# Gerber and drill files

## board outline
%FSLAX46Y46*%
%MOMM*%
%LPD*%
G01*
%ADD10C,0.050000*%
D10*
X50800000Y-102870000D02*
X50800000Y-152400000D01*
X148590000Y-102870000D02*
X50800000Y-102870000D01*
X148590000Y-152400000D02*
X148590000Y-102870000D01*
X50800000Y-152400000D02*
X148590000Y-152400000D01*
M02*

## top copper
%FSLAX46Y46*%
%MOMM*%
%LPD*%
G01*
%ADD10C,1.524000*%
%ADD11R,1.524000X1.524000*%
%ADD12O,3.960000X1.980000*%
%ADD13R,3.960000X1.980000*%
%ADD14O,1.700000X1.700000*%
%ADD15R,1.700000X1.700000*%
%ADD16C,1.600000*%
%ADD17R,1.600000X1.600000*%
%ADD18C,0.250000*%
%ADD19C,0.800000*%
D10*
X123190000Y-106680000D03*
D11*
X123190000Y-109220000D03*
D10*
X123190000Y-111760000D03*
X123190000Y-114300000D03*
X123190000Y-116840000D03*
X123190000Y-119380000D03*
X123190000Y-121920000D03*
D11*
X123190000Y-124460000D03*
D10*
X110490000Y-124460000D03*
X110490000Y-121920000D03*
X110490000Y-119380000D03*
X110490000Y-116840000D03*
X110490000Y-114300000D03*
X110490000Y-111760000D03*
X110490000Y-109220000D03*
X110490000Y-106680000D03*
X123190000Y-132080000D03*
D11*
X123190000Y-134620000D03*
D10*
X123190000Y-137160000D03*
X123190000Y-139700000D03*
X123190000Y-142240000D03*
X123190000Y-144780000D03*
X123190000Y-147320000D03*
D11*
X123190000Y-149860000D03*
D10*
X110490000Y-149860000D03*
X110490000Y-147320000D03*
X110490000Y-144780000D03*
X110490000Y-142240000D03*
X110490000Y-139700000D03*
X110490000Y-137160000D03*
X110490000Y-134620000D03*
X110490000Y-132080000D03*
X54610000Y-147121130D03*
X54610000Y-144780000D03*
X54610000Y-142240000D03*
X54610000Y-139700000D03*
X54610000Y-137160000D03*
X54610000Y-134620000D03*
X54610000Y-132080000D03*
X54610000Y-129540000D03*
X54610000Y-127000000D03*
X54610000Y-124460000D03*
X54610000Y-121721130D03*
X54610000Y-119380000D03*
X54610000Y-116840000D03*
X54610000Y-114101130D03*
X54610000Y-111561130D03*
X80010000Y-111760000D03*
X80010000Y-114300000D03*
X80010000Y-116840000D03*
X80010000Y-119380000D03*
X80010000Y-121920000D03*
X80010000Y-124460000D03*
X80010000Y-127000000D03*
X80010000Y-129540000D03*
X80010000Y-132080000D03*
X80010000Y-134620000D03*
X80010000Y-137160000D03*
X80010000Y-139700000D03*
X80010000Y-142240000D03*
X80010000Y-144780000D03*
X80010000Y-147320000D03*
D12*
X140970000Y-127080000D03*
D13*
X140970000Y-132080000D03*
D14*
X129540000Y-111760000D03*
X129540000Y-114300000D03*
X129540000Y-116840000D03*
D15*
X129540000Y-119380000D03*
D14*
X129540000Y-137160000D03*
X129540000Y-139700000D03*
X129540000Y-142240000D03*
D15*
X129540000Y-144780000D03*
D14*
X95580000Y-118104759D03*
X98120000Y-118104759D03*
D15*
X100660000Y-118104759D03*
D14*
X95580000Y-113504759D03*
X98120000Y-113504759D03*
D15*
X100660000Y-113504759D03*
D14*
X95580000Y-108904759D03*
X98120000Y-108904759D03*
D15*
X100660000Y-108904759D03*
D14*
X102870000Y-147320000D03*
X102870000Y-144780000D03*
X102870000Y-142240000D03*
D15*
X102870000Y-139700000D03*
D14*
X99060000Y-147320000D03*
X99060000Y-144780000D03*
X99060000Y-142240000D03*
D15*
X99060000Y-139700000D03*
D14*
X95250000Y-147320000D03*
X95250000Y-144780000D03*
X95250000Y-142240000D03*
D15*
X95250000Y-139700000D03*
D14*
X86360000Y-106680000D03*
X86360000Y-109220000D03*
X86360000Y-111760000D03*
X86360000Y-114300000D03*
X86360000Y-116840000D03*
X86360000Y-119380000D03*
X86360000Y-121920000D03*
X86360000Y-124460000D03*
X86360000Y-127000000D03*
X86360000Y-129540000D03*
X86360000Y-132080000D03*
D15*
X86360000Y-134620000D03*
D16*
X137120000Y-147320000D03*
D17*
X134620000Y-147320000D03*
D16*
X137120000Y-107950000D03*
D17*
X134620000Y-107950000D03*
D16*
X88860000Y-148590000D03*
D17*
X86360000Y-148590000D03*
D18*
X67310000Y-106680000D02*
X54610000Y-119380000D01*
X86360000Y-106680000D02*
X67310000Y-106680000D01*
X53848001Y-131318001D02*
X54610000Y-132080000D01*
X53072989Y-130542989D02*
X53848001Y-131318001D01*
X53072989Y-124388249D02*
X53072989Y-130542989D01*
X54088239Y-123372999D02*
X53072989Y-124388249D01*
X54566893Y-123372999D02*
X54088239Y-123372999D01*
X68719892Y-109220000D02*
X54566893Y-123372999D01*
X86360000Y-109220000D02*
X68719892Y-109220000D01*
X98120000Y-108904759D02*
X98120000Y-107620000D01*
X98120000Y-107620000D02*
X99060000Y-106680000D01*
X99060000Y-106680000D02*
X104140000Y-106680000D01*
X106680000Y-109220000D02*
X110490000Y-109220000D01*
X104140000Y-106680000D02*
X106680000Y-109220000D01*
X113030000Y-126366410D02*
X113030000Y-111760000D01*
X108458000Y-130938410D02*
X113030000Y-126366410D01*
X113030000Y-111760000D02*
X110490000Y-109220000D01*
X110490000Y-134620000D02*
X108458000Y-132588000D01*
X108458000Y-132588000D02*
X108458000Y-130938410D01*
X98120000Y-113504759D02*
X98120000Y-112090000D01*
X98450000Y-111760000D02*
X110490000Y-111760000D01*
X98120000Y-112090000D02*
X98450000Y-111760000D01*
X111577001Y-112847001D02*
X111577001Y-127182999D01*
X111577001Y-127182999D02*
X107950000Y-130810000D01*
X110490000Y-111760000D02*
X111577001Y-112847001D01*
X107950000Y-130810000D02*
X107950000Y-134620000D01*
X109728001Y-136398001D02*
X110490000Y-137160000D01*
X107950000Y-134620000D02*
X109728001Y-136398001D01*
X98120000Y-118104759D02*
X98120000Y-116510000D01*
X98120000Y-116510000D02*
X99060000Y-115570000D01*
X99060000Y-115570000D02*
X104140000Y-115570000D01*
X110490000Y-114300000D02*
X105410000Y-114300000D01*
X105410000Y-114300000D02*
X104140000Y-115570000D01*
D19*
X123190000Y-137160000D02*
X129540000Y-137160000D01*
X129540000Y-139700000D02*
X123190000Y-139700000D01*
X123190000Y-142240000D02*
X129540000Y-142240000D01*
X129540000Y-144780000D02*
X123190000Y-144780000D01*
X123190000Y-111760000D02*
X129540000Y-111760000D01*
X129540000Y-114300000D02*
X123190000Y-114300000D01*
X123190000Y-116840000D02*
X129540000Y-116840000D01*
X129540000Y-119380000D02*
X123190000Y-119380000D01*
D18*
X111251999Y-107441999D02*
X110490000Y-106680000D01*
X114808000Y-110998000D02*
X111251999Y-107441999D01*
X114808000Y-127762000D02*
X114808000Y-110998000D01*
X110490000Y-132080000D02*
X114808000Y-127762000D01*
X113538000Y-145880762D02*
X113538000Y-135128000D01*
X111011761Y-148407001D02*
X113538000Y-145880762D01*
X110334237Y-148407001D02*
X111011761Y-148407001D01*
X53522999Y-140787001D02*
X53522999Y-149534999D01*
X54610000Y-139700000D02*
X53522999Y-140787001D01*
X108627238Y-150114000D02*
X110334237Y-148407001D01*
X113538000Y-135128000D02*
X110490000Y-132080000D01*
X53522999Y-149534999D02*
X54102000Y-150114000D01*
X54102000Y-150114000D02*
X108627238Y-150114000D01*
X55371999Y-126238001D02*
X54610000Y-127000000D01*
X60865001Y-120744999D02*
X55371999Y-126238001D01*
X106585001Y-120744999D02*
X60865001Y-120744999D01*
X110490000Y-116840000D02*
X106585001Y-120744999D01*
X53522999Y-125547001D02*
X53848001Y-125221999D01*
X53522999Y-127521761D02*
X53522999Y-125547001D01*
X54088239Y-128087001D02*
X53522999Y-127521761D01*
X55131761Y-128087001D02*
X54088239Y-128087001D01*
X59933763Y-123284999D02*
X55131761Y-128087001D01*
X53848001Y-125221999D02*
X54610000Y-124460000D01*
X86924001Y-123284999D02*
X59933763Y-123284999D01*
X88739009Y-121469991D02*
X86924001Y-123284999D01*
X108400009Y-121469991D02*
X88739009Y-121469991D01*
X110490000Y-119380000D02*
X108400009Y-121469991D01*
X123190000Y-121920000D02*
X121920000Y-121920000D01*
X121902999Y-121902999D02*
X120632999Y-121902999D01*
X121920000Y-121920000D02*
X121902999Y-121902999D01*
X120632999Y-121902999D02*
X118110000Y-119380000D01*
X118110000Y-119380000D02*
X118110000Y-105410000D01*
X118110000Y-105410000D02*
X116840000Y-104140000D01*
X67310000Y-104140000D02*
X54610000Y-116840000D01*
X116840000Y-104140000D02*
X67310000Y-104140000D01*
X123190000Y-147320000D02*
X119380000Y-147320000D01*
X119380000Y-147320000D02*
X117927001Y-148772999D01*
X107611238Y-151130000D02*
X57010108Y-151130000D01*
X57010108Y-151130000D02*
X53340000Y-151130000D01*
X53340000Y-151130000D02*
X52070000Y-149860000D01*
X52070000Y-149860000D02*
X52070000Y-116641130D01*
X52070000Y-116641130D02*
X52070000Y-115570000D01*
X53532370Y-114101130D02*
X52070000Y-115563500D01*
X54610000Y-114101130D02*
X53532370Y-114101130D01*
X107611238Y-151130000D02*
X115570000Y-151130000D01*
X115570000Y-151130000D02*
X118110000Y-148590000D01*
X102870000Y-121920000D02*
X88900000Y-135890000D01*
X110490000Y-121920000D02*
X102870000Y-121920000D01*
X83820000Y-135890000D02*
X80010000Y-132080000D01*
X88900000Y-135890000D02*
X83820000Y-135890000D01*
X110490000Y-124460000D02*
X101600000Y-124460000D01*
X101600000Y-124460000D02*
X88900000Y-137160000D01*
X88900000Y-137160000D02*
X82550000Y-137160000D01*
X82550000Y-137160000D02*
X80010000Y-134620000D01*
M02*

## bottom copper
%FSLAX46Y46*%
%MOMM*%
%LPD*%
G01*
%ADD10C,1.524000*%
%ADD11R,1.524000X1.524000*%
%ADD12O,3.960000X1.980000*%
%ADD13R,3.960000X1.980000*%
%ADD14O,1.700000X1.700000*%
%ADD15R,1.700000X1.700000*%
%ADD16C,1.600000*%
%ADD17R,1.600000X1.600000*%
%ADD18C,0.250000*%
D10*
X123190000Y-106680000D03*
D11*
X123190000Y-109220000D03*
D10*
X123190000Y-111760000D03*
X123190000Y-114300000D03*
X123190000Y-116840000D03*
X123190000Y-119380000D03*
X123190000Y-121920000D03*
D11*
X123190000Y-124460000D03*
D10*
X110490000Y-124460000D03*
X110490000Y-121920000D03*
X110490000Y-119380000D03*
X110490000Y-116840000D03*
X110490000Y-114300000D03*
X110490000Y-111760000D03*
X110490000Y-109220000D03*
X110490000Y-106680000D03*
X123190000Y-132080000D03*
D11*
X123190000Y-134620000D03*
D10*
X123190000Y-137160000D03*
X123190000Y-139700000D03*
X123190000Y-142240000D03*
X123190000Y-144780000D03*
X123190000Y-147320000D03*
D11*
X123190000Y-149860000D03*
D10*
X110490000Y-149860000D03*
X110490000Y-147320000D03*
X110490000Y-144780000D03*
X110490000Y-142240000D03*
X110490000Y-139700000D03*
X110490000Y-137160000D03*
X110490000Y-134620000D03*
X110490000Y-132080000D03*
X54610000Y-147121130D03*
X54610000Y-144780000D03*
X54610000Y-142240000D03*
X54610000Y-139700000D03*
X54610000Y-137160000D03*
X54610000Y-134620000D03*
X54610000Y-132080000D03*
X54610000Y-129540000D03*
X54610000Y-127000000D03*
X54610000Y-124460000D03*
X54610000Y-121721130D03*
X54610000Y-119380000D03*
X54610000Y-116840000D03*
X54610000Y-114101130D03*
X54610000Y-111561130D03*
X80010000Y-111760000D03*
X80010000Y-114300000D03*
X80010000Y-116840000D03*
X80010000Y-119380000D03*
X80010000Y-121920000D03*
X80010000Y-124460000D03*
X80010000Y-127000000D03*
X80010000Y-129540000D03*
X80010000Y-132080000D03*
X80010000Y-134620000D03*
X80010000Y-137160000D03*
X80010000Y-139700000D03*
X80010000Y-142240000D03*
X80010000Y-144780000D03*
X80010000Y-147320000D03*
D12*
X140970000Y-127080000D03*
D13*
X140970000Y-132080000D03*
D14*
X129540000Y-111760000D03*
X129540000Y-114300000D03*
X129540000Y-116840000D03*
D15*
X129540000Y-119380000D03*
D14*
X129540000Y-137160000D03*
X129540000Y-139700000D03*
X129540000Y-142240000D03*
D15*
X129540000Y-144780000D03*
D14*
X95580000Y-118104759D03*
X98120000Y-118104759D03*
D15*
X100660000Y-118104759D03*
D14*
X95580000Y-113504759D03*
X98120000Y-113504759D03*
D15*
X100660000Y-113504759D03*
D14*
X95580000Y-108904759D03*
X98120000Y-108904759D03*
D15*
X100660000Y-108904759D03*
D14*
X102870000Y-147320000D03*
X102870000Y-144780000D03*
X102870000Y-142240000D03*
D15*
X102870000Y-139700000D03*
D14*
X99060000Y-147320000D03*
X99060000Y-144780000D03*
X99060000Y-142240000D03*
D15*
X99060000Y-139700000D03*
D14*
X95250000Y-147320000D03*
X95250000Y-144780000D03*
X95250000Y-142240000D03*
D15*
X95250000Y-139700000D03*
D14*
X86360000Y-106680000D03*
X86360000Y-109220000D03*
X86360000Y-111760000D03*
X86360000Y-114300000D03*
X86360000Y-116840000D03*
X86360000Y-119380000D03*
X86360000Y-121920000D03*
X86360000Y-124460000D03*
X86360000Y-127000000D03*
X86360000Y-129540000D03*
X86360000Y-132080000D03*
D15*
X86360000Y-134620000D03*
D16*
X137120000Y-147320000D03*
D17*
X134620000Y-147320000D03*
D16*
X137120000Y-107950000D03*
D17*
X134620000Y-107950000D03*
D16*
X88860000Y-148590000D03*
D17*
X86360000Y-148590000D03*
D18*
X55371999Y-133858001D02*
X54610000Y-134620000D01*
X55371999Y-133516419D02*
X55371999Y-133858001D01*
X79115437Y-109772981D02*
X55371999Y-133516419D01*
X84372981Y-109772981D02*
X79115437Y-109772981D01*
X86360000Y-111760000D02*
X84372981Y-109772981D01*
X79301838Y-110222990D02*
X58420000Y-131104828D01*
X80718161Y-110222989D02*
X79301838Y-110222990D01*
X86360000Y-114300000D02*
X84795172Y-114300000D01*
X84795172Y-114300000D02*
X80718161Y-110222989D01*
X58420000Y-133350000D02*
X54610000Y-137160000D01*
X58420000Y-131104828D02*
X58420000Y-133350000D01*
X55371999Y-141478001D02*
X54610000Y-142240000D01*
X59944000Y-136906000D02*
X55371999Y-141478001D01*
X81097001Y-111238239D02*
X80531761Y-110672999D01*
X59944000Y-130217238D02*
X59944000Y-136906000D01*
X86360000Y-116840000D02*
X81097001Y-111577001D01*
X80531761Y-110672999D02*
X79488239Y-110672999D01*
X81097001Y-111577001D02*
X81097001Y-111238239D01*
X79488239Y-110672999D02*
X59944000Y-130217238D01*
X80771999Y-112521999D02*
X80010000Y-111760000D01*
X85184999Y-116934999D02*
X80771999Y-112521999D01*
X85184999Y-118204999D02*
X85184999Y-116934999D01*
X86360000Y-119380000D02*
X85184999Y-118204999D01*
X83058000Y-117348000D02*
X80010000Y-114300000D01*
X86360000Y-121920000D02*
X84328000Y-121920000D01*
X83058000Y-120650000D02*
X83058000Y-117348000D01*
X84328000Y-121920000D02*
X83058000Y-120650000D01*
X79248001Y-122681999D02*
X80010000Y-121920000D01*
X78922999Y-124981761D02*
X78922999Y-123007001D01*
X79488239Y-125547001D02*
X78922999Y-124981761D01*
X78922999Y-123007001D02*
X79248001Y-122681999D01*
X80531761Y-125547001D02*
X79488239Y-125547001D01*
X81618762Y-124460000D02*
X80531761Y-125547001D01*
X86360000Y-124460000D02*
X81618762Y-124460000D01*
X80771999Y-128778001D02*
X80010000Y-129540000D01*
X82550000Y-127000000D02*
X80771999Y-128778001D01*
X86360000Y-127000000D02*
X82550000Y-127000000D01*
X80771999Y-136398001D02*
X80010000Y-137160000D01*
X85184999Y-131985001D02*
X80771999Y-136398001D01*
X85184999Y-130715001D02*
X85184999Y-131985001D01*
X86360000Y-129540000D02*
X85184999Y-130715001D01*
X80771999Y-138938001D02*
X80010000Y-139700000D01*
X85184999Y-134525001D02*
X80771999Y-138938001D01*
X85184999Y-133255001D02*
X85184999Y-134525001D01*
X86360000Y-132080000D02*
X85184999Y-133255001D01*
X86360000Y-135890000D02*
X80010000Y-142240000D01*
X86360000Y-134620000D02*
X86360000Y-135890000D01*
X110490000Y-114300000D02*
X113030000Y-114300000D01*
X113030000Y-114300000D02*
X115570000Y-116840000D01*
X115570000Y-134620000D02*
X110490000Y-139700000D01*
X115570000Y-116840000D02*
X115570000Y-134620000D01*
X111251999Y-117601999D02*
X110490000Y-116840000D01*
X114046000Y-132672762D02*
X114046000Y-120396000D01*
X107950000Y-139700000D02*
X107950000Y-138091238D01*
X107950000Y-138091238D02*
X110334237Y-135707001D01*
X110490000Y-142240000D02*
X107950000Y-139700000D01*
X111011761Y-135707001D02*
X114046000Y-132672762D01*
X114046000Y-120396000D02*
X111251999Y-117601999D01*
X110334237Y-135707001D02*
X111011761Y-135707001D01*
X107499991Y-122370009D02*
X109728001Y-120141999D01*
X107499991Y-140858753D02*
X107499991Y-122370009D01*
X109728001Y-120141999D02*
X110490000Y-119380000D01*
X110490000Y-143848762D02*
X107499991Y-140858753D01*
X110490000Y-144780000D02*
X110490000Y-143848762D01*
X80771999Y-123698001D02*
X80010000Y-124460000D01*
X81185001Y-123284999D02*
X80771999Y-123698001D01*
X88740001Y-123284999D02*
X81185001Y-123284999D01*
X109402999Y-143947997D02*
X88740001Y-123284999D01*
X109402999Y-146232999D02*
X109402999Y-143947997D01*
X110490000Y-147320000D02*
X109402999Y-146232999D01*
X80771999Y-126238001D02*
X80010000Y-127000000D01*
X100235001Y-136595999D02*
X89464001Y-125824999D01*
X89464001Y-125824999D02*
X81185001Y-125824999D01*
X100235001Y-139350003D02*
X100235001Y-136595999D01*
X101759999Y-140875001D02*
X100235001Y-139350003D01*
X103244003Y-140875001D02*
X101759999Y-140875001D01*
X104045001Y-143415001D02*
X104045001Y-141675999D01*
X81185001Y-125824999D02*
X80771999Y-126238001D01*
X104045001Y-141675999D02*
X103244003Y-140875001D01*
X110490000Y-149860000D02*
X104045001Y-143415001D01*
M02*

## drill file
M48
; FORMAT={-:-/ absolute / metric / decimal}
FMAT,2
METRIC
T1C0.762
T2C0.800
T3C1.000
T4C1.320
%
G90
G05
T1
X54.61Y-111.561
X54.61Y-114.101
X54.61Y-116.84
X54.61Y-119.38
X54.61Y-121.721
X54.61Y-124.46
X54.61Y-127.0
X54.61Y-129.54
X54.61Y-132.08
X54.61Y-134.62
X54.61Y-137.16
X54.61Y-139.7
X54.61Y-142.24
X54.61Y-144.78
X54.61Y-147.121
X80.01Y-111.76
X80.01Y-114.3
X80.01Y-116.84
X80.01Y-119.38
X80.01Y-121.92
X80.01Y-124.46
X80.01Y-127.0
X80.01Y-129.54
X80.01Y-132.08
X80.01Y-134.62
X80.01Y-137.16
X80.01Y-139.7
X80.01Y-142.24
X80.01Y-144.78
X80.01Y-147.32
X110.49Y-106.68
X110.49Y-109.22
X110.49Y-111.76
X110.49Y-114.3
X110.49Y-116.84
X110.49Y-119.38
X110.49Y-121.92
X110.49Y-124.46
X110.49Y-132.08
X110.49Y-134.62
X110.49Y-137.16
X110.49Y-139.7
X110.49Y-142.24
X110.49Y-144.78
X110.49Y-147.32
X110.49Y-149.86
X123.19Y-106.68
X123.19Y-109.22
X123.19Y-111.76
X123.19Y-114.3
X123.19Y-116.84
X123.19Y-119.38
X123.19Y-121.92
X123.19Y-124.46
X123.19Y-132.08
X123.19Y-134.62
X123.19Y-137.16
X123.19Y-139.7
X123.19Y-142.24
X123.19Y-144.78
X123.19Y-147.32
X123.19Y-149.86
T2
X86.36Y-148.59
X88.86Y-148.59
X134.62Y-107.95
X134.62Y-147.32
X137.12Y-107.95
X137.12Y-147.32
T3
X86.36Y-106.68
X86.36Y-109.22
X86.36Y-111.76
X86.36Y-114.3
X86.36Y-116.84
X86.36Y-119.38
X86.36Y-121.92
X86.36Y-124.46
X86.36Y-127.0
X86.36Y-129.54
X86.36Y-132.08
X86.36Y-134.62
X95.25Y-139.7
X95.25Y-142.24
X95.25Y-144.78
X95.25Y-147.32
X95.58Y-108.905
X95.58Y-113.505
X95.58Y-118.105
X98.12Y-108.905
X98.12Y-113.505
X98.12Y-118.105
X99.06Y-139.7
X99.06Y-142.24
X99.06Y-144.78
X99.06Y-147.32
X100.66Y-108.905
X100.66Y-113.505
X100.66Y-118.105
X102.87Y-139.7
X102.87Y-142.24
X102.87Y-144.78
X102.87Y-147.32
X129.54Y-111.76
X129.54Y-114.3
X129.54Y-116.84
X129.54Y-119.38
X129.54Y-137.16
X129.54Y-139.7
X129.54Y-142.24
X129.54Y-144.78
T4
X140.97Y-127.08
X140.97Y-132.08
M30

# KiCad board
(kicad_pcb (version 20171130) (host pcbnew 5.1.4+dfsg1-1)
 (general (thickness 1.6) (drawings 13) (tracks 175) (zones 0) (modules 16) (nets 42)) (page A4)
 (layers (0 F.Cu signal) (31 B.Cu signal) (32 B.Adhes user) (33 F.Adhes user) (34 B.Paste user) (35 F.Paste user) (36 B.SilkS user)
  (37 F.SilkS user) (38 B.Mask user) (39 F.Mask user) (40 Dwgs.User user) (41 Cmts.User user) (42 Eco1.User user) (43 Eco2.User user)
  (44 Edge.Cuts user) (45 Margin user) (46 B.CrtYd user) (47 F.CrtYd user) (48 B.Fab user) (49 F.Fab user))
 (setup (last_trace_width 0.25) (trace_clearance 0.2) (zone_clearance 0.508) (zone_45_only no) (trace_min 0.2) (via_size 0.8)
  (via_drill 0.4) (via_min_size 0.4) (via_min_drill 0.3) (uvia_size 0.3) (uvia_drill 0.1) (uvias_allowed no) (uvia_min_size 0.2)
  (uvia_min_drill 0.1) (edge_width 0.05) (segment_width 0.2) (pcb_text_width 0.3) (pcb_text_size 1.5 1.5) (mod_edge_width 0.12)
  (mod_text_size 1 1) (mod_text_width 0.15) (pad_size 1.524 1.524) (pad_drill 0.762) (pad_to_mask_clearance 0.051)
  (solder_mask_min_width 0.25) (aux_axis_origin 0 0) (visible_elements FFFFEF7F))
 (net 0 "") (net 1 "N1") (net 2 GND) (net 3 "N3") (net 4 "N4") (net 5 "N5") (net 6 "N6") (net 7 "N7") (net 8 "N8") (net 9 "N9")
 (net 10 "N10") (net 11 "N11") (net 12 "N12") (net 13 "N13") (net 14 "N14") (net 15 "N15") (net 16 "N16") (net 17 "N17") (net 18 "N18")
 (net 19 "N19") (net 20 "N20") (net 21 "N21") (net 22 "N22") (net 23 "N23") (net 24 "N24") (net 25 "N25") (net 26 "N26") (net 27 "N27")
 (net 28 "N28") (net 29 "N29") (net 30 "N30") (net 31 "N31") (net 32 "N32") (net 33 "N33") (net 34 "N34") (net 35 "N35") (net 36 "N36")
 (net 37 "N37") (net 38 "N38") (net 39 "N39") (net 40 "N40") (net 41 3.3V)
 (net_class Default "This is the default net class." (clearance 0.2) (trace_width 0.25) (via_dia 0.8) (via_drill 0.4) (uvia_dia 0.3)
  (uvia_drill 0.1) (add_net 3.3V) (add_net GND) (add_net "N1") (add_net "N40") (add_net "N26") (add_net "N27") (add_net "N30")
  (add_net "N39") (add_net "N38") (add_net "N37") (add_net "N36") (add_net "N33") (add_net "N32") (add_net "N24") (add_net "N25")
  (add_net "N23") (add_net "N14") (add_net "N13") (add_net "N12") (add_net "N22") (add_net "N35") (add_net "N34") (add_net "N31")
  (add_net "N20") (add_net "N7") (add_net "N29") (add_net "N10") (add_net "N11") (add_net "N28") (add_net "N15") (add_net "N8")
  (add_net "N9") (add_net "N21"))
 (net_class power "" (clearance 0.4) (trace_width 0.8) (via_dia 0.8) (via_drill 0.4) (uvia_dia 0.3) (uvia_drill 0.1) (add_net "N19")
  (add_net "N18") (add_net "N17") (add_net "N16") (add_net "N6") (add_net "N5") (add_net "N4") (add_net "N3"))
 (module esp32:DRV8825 (layer F.Cu) (at 116.84 115.57)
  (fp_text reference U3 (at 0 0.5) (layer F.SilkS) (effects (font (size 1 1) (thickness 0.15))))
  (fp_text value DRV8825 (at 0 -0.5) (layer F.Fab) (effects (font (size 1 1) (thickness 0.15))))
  (pad 16 thru_hole circle (at 6.35 -8.89) (size 1.524 1.524) (drill 0.762) (layers *.Cu *.Mask) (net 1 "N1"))
  (pad 15 thru_hole rect (at 6.35 -6.35) (size 1.524 1.524) (drill 0.762) (layers *.Cu *.Mask) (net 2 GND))
  (pad 14 thru_hole circle (at 6.35 -3.81) (size 1.524 1.524) (drill 0.762) (layers *.Cu *.Mask) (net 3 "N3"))
  (pad 13 thru_hole circle (at 6.35 -1.27) (size 1.524 1.524) (drill 0.762) (layers *.Cu *.Mask) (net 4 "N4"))
  (pad 12 thru_hole circle (at 6.35 1.27) (size 1.524 1.524) (drill 0.762) (layers *.Cu *.Mask) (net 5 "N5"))
  (pad 11 thru_hole circle (at 6.35 3.81) (size 1.524 1.524) (drill 0.762) (layers *.Cu *.Mask) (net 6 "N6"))
  (pad 10 thru_hole circle (at 6.35 6.35) (size 1.524 1.524) (drill 0.762) (layers *.Cu *.Mask) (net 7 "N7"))
  (pad 9 thru_hole rect (at 6.35 8.89) (size 1.524 1.524) (drill 0.762) (layers *.Cu *.Mask) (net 2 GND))
  (pad 8 thru_hole circle (at -6.35 8.89) (size 1.524 1.524) (drill 0.762) (layers *.Cu *.Mask) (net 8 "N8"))
  (pad 7 thru_hole circle (at -6.35 6.35) (size 1.524 1.524) (drill 0.762) (layers *.Cu *.Mask) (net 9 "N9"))
  (pad 6 thru_hole circle (at -6.35 3.81) (size 1.524 1.524) (drill 0.762) (layers *.Cu *.Mask) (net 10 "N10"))
  (pad 5 thru_hole circle (at -6.35 1.27) (size 1.524 1.524) (drill 0.762) (layers *.Cu *.Mask) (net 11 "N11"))
  (pad 4 thru_hole circle (at -6.35 -1.27) (size 1.524 1.524) (drill 0.762) (layers *.Cu *.Mask) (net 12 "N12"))
  (pad 3 thru_hole circle (at -6.35 -3.81) (size 1.524 1.524) (drill 0.762) (layers *.Cu *.Mask) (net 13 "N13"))
  (pad 2 thru_hole circle (at -6.35 -6.35) (size 1.524 1.524) (drill 0.762) (layers *.Cu *.Mask) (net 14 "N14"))
  (pad 1 thru_hole circle (at -6.35 -8.89) (size 1.524 1.524) (drill 0.762) (layers *.Cu *.Mask) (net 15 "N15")))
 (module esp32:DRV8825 (layer F.Cu) (at 116.84 140.97)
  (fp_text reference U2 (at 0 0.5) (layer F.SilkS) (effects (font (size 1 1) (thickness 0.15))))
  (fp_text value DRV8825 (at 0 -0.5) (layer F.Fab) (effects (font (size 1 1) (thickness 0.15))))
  (pad 16 thru_hole circle (at 6.35 -8.89) (size 1.524 1.524) (drill 0.762) (layers *.Cu *.Mask) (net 1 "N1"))
  (pad 15 thru_hole rect (at 6.35 -6.35) (size 1.524 1.524) (drill 0.762) (layers *.Cu *.Mask) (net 2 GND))
  (pad 14 thru_hole circle (at 6.35 -3.81) (size 1.524 1.524) (drill 0.762) (layers *.Cu *.Mask) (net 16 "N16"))
  (pad 13 thru_hole circle (at 6.35 -1.27) (size 1.524 1.524) (drill 0.762) (layers *.Cu *.Mask) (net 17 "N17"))
  (pad 12 thru_hole circle (at 6.35 1.27) (size 1.524 1.524) (drill 0.762) (layers *.Cu *.Mask) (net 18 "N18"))
  (pad 11 thru_hole circle (at 6.35 3.81) (size 1.524 1.524) (drill 0.762) (layers *.Cu *.Mask) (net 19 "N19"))
  (pad 10 thru_hole circle (at 6.35 6.35) (size 1.524 1.524) (drill 0.762) (layers *.Cu *.Mask) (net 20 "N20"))
  (pad 9 thru_hole rect (at 6.35 8.89) (size 1.524 1.524) (drill 0.762) (layers *.Cu *.Mask) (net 2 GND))
  (pad 8 thru_hole circle (at -6.35 8.89) (size 1.524 1.524) (drill 0.762) (layers *.Cu *.Mask) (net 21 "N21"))
  (pad 7 thru_hole circle (at -6.35 6.35) (size 1.524 1.524) (drill 0.762) (layers *.Cu *.Mask) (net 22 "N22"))
  (pad 6 thru_hole circle (at -6.35 3.81) (size 1.524 1.524) (drill 0.762) (layers *.Cu *.Mask) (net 10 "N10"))
  (pad 5 thru_hole circle (at -6.35 1.27) (size 1.524 1.524) (drill 0.762) (layers *.Cu *.Mask) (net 11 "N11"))
  (pad 4 thru_hole circle (at -6.35 -1.27) (size 1.524 1.524) (drill 0.762) (layers *.Cu *.Mask) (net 12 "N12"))
  (pad 3 thru_hole circle (at -6.35 -3.81) (size 1.524 1.524) (drill 0.762) (layers *.Cu *.Mask) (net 13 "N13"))
  (pad 2 thru_hole circle (at -6.35 -6.35) (size 1.524 1.524) (drill 0.762) (layers *.Cu *.Mask) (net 14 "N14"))
  (pad 1 thru_hole circle (at -6.35 -8.89) (size 1.524 1.524) (drill 0.762) (layers *.Cu *.Mask) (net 15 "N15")))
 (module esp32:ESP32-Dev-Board (layer F.Cu) (at 67.31 129.54 90)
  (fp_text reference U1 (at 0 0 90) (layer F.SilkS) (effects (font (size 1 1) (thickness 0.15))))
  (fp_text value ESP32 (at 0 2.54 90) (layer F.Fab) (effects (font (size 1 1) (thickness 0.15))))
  (pad 30 thru_hole circle (at -17.58113 -12.7 90) (size 1.524 1.524) (drill 0.762) (layers *.Cu *.Mask) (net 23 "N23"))
  (pad 29 thru_hole circle (at -15.24 -12.7 90) (size 1.524 1.524) (drill 0.762) (layers *.Cu *.Mask) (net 2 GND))
  (pad 28 thru_hole circle (at -12.7 -12.7 90) (size 1.524 1.524) (drill 0.762) (layers *.Cu *.Mask) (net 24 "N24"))
  (pad 27 thru_hole circle (at -10.16 -12.7 90) (size 1.524 1.524) (drill 0.762) (layers *.Cu *.Mask) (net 15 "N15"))
  (pad 26 thru_hole circle (at -7.62 -12.7 90) (size 1.524 1.524) (drill 0.762) (layers *.Cu *.Mask) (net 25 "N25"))
  (pad 25 thru_hole circle (at -5.08 -12.7 90) (size 1.524 1.524) (drill 0.762) (layers *.Cu *.Mask) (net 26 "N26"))
  (pad 24 thru_hole circle (at -2.54 -12.7 90) (size 1.524 1.524) (drill 0.762) (layers *.Cu *.Mask) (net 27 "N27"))
  (pad 23 thru_hole circle (at 0 -12.7 90) (size 1.524 1.524) (drill 0.762) (layers *.Cu *.Mask) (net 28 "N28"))
  (pad 22 thru_hole circle (at 2.54 -12.7 90) (size 1.524 1.524) (drill 0.762) (layers *.Cu *.Mask) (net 11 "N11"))
  (pad 21 thru_hole circle (at 5.08 -12.7 90) (size 1.524 1.524) (drill 0.762) (layers *.Cu *.Mask) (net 10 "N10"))
  (pad 20 thru_hole circle (at 7.81887 -12.7 90) (size 1.524 1.524) (drill 0.762) (layers *.Cu *.Mask) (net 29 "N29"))
  (pad 19 thru_hole circle (at 10.16 -12.7 90) (size 1.524 1.524) (drill 0.762) (layers *.Cu *.Mask) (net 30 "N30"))
  (pad 18 thru_hole circle (at 12.7 -12.7 90) (size 1.524 1.524) (drill 0.762) (layers *.Cu *.Mask) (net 7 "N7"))
  (pad 17 thru_hole circle (at 15.43887 -12.7 90) (size 1.524 1.524) (drill 0.762) (layers *.Cu *.Mask) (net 20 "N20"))
  (pad 16 thru_hole circle (at 17.97887 -12.7 90) (size 1.524 1.524) (drill 0.762) (layers *.Cu *.Mask) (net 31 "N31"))
  (pad 15 thru_hole circle (at 17.78 12.7 90) (size 1.524 1.524) (drill 0.762) (layers *.Cu *.Mask) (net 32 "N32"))
  (pad 14 thru_hole circle (at 15.24 12.7 90) (size 1.524 1.524) (drill 0.762) (layers *.Cu *.Mask) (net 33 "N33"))
  (pad 13 thru_hole circle (at 12.7 12.7 90) (size 1.524 1.524) (drill 0.762) (layers *.Cu *.Mask) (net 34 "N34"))
  (pad 12 thru_hole circle (at 10.16 12.7 90) (size 1.524 1.524) (drill 0.762) (layers *.Cu *.Mask) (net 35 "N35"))
  (pad 11 thru_hole circle (at 7.62 12.7 90) (size 1.524 1.524) (drill 0.762) (layers *.Cu *.Mask) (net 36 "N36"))
  (pad 10 thru_hole circle (at 5.08 12.7 90) (size 1.524 1.524) (drill 0.762) (layers *.Cu *.Mask) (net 22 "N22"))
  (pad 9 thru_hole circle (at 2.54 12.7 90) (size 1.524 1.524) (drill 0.762) (layers *.Cu *.Mask) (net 21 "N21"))
  (pad 8 thru_hole circle (at 0 12.7 90) (size 1.524 1.524) (drill 0.762) (layers *.Cu *.Mask) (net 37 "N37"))
  (pad 7 thru_hole circle (at -2.54 12.7 90) (size 1.524 1.524) (drill 0.762) (layers *.Cu *.Mask) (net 9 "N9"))
  (pad 6 thru_hole circle (at -5.08 12.7 90) (size 1.524 1.524) (drill 0.762) (layers *.Cu *.Mask) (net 8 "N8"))
  (pad 5 thru_hole circle (at -7.62 12.7 90) (size 1.524 1.524) (drill 0.762) (layers *.Cu *.Mask) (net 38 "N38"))
  (pad 4 thru_hole circle (at -10.16 12.7 90) (size 1.524 1.524) (drill 0.762) (layers *.Cu *.Mask) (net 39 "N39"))
  (pad 3 thru_hole circle (at -12.7 12.7 90) (size 1.524 1.524) (drill 0.762) (layers *.Cu *.Mask) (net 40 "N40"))
  (pad 2 thru_hole circle (at -15.24 12.7 90) (size 1.524 1.524) (drill 0.762) (layers *.Cu *.Mask) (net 2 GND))
  (pad 1 thru_hole circle (at -17.78 12.7 90) (size 1.524 1.524) (drill 0.762) (layers *.Cu *.Mask) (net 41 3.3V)))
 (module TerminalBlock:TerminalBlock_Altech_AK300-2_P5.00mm (layer F.Cu) (at 140.97 132.08 90)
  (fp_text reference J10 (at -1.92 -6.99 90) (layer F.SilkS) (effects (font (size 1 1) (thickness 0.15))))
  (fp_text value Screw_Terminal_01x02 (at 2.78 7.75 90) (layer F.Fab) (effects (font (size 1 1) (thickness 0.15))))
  (pad 2 thru_hole oval (at 5 0 90) (size 1.98 3.96) (drill 1.32) (layers *.Cu *.Mask) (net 1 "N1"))
  (pad 1 thru_hole rect (at 0 0 90) (size 1.98 3.96) (drill 1.32) (layers *.Cu *.Mask) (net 2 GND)))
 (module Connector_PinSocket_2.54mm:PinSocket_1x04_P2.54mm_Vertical (layer F.Cu) (at 129.54 119.38 180)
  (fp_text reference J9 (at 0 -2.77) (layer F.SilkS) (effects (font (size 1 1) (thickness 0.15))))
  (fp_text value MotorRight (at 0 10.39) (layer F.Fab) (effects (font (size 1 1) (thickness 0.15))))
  (pad 4 thru_hole oval (at 0 7.62 180) (size 1.7 1.7) (drill 1) (layers *.Cu *.Mask) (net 3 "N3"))
  (pad 3 thru_hole oval (at 0 5.08 180) (size 1.7 1.7) (drill 1) (layers *.Cu *.Mask) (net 4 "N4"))
  (pad 2 thru_hole oval (at 0 2.54 180) (size 1.7 1.7) (drill 1) (layers *.Cu *.Mask) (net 5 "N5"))
  (pad 1 thru_hole rect (at 0 0 180) (size 1.7 1.7) (drill 1) (layers *.Cu *.Mask) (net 6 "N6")))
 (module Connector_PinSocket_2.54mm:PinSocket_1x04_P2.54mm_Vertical (layer F.Cu) (at 129.54 144.78 180)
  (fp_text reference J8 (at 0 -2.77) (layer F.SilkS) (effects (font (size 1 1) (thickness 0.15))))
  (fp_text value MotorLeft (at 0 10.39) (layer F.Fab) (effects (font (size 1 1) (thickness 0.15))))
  (pad 4 thru_hole oval (at 0 7.62 180) (size 1.7 1.7) (drill 1) (layers *.Cu *.Mask) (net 16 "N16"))
  (pad 3 thru_hole oval (at 0 5.08 180) (size 1.7 1.7) (drill 1) (layers *.Cu *.Mask) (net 17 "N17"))
  (pad 2 thru_hole oval (at 0 2.54 180) (size 1.7 1.7) (drill 1) (layers *.Cu *.Mask) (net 18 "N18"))
  (pad 1 thru_hole rect (at 0 0 180) (size 1.7 1.7) (drill 1) (layers *.Cu *.Mask) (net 19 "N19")))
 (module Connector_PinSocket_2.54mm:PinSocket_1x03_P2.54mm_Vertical (layer F.Cu) (at 100.66 118.104759 270)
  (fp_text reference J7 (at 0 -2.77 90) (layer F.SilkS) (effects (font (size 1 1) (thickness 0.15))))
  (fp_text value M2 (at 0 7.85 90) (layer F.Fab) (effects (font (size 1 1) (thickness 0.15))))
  (pad 3 thru_hole oval (at 0 5.08 270) (size 1.7 1.7) (drill 1) (layers *.Cu *.Mask) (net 41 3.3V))
  (pad 2 thru_hole oval (at 0 2.54 270) (size 1.7 1.7) (drill 1) (layers *.Cu *.Mask) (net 12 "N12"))
  (pad 1 thru_hole rect (at 0 0 270) (size 1.7 1.7) (drill 1) (layers *.Cu *.Mask) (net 2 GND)))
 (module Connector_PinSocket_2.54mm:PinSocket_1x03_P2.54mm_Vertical (layer F.Cu) (at 100.66 113.504759 270)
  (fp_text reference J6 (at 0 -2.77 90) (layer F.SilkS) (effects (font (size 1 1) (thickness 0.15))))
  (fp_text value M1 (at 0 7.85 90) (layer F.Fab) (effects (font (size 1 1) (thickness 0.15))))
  (pad 3 thru_hole oval (at 0 5.08 270) (size 1.7 1.7) (drill 1) (layers *.Cu *.Mask) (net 41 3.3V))
  (pad 2 thru_hole oval (at 0 2.54 270) (size 1.7 1.7) (drill 1) (layers *.Cu *.Mask) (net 13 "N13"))
  (pad 1 thru_hole rect (at 0 0 270) (size 1.7 1.7) (drill 1) (layers *.Cu *.Mask) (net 2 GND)))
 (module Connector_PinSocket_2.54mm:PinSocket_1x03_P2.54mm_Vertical (layer F.Cu) (at 100.66 108.904759 270)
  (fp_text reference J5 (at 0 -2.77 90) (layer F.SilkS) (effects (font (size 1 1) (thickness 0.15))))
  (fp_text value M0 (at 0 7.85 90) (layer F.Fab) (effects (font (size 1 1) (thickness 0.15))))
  (pad 3 thru_hole oval (at 0 5.08 270) (size 1.7 1.7) (drill 1) (layers *.Cu *.Mask) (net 41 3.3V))
  (pad 2 thru_hole oval (at 0 2.54 270) (size 1.7 1.7) (drill 1) (layers *.Cu *.Mask) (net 14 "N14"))
  (pad 1 thru_hole rect (at 0 0 270) (size 1.7 1.7) (drill 1) (layers *.Cu *.Mask) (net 2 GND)))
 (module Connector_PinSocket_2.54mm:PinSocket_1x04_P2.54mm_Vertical (layer F.Cu) (at 102.87 139.7)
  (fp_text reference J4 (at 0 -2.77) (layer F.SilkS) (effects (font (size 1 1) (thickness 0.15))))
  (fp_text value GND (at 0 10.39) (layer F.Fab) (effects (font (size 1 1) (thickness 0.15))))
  (pad 4 thru_hole oval (at 0 7.62) (size 1.7 1.7) (drill 1) (layers *.Cu *.Mask) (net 2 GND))
  (pad 3 thru_hole oval (at 0 5.08) (size 1.7 1.7) (drill 1) (layers *.Cu *.Mask) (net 2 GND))
  (pad 2 thru_hole oval (at 0 2.54) (size 1.7 1.7) (drill 1) (layers *.Cu *.Mask) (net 2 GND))
  (pad 1 thru_hole rect (at 0 0) (size 1.7 1.7) (drill 1) (layers *.Cu *.Mask) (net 2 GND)))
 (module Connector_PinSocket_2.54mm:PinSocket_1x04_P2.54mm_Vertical (layer F.Cu) (at 99.06 139.7)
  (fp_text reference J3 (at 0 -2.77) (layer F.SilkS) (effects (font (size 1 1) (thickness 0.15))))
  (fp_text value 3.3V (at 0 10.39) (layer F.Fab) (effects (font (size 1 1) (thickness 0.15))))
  (pad 4 thru_hole oval (at 0 7.62) (size 1.7 1.7) (drill 1) (layers *.Cu *.Mask) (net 41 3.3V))
  (pad 3 thru_hole oval (at 0 5.08) (size 1.7 1.7) (drill 1) (layers *.Cu *.Mask) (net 41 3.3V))
  (pad 2 thru_hole oval (at 0 2.54) (size 1.7 1.7) (drill 1) (layers *.Cu *.Mask) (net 41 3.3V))
  (pad 1 thru_hole rect (at 0 0) (size 1.7 1.7) (drill 1) (layers *.Cu *.Mask) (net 41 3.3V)))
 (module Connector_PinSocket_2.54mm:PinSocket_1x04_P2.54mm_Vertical (layer F.Cu) (at 95.25 139.7)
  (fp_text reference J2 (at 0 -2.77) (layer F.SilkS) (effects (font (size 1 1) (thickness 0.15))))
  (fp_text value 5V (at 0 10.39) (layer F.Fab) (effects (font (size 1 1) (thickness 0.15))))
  (pad 4 thru_hole oval (at 0 7.62) (size 1.7 1.7) (drill 1) (layers *.Cu *.Mask) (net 23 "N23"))
  (pad 3 thru_hole oval (at 0 5.08) (size 1.7 1.7) (drill 1) (layers *.Cu *.Mask) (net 23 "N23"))
  (pad 2 thru_hole oval (at 0 2.54) (size 1.7 1.7) (drill 1) (layers *.Cu *.Mask) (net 23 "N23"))
  (pad 1 thru_hole rect (at 0 0) (size 1.7 1.7) (drill 1) (layers *.Cu *.Mask) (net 23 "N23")))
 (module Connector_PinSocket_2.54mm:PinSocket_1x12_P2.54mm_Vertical (layer F.Cu) (at 86.36 134.62 180)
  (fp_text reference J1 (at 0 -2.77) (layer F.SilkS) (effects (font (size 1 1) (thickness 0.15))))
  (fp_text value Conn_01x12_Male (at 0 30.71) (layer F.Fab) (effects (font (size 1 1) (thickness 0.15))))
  (pad 12 thru_hole oval (at 0 27.94 180) (size 1.7 1.7) (drill 1) (layers *.Cu *.Mask) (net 30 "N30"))
  (pad 11 thru_hole oval (at 0 25.4 180) (size 1.7 1.7) (drill 1) (layers *.Cu *.Mask) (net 27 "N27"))
  (pad 10 thru_hole oval (at 0 22.86 180) (size 1.7 1.7) (drill 1) (layers *.Cu *.Mask) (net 26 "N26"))
  (pad 9 thru_hole oval (at 0 20.32 180) (size 1.7 1.7) (drill 1) (layers *.Cu *.Mask) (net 25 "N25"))
  (pad 8 thru_hole oval (at 0 17.78 180) (size 1.7 1.7) (drill 1) (layers *.Cu *.Mask) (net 24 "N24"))
  (pad 7 thru_hole oval (at 0 15.24 180) (size 1.7 1.7) (drill 1) (layers *.Cu *.Mask) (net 32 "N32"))
  (pad 6 thru_hole oval (at 0 12.7 180) (size 1.7 1.7) (drill 1) (layers *.Cu *.Mask) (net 33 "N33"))
  (pad 5 thru_hole oval (at 0 10.16 180) (size 1.7 1.7) (drill 1) (layers *.Cu *.Mask) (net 36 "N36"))
  (pad 4 thru_hole oval (at 0 7.62 180) (size 1.7 1.7) (drill 1) (layers *.Cu *.Mask) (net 37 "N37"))
  (pad 3 thru_hole oval (at 0 5.08 180) (size 1.7 1.7) (drill 1) (layers *.Cu *.Mask) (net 38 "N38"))
  (pad 2 thru_hole oval (at 0 2.54 180) (size 1.7 1.7) (drill 1) (layers *.Cu *.Mask) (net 39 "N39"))
  (pad 1 thru_hole rect (at 0 0 180) (size 1.7 1.7) (drill 1) (layers *.Cu *.Mask) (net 40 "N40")))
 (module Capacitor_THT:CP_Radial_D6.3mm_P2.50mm (layer F.Cu) (at 134.62 147.32)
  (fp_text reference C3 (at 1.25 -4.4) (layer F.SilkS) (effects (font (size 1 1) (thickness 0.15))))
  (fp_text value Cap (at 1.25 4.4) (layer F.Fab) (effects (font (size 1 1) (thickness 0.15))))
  (pad 2 thru_hole circle (at 2.5 0) (size 1.6 1.6) (drill 0.8) (layers *.Cu *.Mask) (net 2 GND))
  (pad 1 thru_hole rect (at 0 0) (size 1.6 1.6) (drill 0.8) (layers *.Cu *.Mask) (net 1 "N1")))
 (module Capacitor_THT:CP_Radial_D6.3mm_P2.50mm (layer F.Cu) (at 134.62 107.95)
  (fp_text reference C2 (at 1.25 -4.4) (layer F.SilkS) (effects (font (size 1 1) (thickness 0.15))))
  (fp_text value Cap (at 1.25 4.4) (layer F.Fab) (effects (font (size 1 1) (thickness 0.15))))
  (pad 2 thru_hole circle (at 2.5 0) (size 1.6 1.6) (drill 0.8) (layers *.Cu *.Mask) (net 2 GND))
  (pad 1 thru_hole rect (at 0 0) (size 1.6 1.6) (drill 0.8) (layers *.Cu *.Mask) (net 1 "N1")))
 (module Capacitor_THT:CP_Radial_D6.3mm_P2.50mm (layer F.Cu) (at 86.36 148.59)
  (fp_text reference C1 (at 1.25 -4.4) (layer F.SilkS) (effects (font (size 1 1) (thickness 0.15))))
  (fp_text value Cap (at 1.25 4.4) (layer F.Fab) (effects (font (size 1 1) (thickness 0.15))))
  (pad 2 thru_hole circle (at 2.5 0) (size 1.6 1.6) (drill 0.8) (layers *.Cu *.Mask) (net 2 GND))
  (pad 1 thru_hole rect (at 0 0) (size 1.6 1.6) (drill 0.8) (layers *.Cu *.Mask) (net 41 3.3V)))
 (gr_line (start 50.8 102.87) (end 50.8 152.4) (layer Edge.Cuts) (width 0.05))
 (gr_line (start 148.59 102.87) (end 50.8 102.87) (layer Edge.Cuts) (width 0.05))
 (gr_line (start 148.59 152.4) (end 148.59 102.87) (layer Edge.Cuts) (width 0.05))
 (gr_line (start 50.8 152.4) (end 148.59 152.4) (layer Edge.Cuts) (width 0.05))
 (segment (start 67.31 106.68) (end 54.61 119.38) (width 0.25) (layer F.Cu) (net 30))
 (segment (start 86.36 106.68) (end 67.31 106.68) (width 0.25) (layer F.Cu) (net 30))
 (segment (start 53.848001 131.318001) (end 54.61 132.08) (width 0.25) (layer F.Cu) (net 27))
 (segment (start 53.072989 130.542989) (end 53.848001 131.318001) (width 0.25) (layer F.Cu) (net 27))
 (segment (start 53.072989 124.388249) (end 53.072989 130.542989) (width 0.25) (layer F.Cu) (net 27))
 (segment (start 54.088239 123.372999) (end 53.072989 124.388249) (width 0.25) (layer F.Cu) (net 27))
 (segment (start 54.566893 123.372999) (end 54.088239 123.372999) (width 0.25) (layer F.Cu) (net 27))
 (segment (start 68.719892 109.22) (end 54.566893 123.372999) (width 0.25) (layer F.Cu) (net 27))
 (segment (start 86.36 109.22) (end 68.719892 109.22) (width 0.25) (layer F.Cu) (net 27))
 (segment (start 55.371999 133.858001) (end 54.61 134.62) (width 0.25) (layer B.Cu) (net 26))
 (segment (start 55.371999 133.516419) (end 55.371999 133.858001) (width 0.25) (layer B.Cu) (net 26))
 (segment (start 79.115437 109.772981) (end 55.371999 133.516419) (width 0.25) (layer B.Cu) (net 26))
 (segment (start 84.372981 109.772981) (end 79.115437 109.772981) (width 0.25) (layer B.Cu) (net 26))
 (segment (start 86.36 111.76) (end 84.372981 109.772981) (width 0.25) (layer B.Cu) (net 26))
 (segment (start 79.301838 110.22299) (end 58.42 131.104828) (width 0.25) (layer B.Cu) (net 25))
 (segment (start 80.718161 110.222989) (end 79.301838 110.22299) (width 0.25) (layer B.Cu) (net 25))
 (segment (start 86.36 114.3) (end 84.795172 114.3) (width 0.25) (layer B.Cu) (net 25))
 (segment (start 84.795172 114.3) (end 80.718161 110.222989) (width 0.25) (layer B.Cu) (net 25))
 (segment (start 58.42 133.35) (end 54.61 137.16) (width 0.25) (layer B.Cu) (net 25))
 (segment (start 58.42 131.104828) (end 58.42 133.35) (width 0.25) (layer B.Cu) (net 25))
 (segment (start 55.371999 141.478001) (end 54.61 142.24) (width 0.25) (layer B.Cu) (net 24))
 (segment (start 59.944 136.906) (end 55.371999 141.478001) (width 0.25) (layer B.Cu) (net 24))
 (segment (start 81.097001 111.238239) (end 80.531761 110.672999) (width 0.25) (layer B.Cu) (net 24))
 (segment (start 59.944 130.217238) (end 59.944 136.906) (width 0.25) (layer B.Cu) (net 24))
 (segment (start 86.36 116.84) (end 81.097001 111.577001) (width 0.25) (layer B.Cu) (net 24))
 (segment (start 80.531761 110.672999) (end 79.488239 110.672999) (width 0.25) (layer B.Cu) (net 24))
 (segment (start 81.097001 111.577001) (end 81.097001 111.238239) (width 0.25) (layer B.Cu) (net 24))
 (segment (start 79.488239 110.672999) (end 59.944 130.217238) (width 0.25) (layer B.Cu) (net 24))
 (segment (start 80.771999 112.521999) (end 80.01 111.76) (width 0.25) (layer B.Cu) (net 32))
 (segment (start 85.184999 116.934999) (end 80.771999 112.521999) (width 0.25) (layer B.Cu) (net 32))
 (segment (start 85.184999 118.204999) (end 85.184999 116.934999) (width 0.25) (layer B.Cu) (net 32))
 (segment (start 86.36 119.38) (end 85.184999 118.204999) (width 0.25) (layer B.Cu) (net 32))
 (segment (start 83.058 117.348) (end 80.01 114.3) (width 0.25) (layer B.Cu) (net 33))
 (segment (start 86.36 121.92) (end 84.328 121.92) (width 0.25) (layer B.Cu) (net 33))
 (segment (start 83.058 120.65) (end 83.058 117.348) (width 0.25) (layer B.Cu) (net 33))
 (segment (start 84.328 121.92) (end 83.058 120.65) (width 0.25) (layer B.Cu) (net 33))
 (segment (start 79.248001 122.681999) (end 80.01 121.92) (width 0.25) (layer B.Cu) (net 36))
 (segment (start 78.922999 124.981761) (end 78.922999 123.007001) (width 0.25) (layer B.Cu) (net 36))
 (segment (start 79.488239 125.547001) (end 78.922999 124.981761) (width 0.25) (layer B.Cu) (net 36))
 (segment (start 78.922999 123.007001) (end 79.248001 122.681999) (width 0.25) (layer B.Cu) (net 36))
 (segment (start 80.531761 125.547001) (end 79.488239 125.547001) (width 0.25) (layer B.Cu) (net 36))
 (segment (start 81.618762 124.46) (end 80.531761 125.547001) (width 0.25) (layer B.Cu) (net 36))
 (segment (start 86.36 124.46) (end 81.618762 124.46) (width 0.25) (layer B.Cu) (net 36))
 (segment (start 80.771999 128.778001) (end 80.01 129.54) (width 0.25) (layer B.Cu) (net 37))
 (segment (start 82.55 127) (end 80.771999 128.778001) (width 0.25) (layer B.Cu) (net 37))
 (segment (start 86.36 127) (end 82.55 127) (width 0.25) (layer B.Cu) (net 37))
 (segment (start 80.771999 136.398001) (end 80.01 137.16) (width 0.25) (layer B.Cu) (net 38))
 (segment (start 85.184999 131.985001) (end 80.771999 136.398001) (width 0.25) (layer B.Cu) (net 38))
 (segment (start 85.184999 130.715001) (end 85.184999 131.985001) (width 0.25) (layer B.Cu) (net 38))
 (segment (start 86.36 129.54) (end 85.184999 130.715001) (width 0.25) (layer B.Cu) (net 38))
 (segment (start 80.771999 138.938001) (end 80.01 139.7) (width 0.25) (layer B.Cu) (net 39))
 (segment (start 85.184999 134.525001) (end 80.771999 138.938001) (width 0.25) (layer B.Cu) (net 39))
 (segment (start 85.184999 133.255001) (end 85.184999 134.525001) (width 0.25) (layer B.Cu) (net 39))
 (segment (start 86.36 132.08) (end 85.184999 133.255001) (width 0.25) (layer B.Cu) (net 39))
 (segment (start 86.36 135.89) (end 80.01 142.24) (width 0.25) (layer B.Cu) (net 40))
 (segment (start 86.36 134.62) (end 86.36 135.89) (width 0.25) (layer B.Cu) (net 40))
 (segment (start 98.12 108.904759) (end 98.12 107.62) (width 0.25) (layer F.Cu) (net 14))
 (segment (start 98.12 107.62) (end 99.06 106.68) (width 0.25) (layer F.Cu) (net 14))
 (segment (start 99.06 106.68) (end 104.14 106.68) (width 0.25) (layer F.Cu) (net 14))
 (segment (start 106.68 109.22) (end 110.49 109.22) (width 0.25) (layer F.Cu) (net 14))
 (segment (start 104.14 106.68) (end 106.68 109.22) (width 0.25) (layer F.Cu) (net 14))
 (segment (start 113.03 126.36641) (end 113.03 111.76) (width 0.25) (layer F.Cu) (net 14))
 (segment (start 108.458 130.93841) (end 113.03 126.36641) (width 0.25) (layer F.Cu) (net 14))
 (segment (start 113.03 111.76) (end 110.49 109.22) (width 0.25) (layer F.Cu) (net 14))
 (segment (start 110.49 134.62) (end 108.458 132.588) (width 0.25) (layer F.Cu) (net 14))
 (segment (start 108.458 132.588) (end 108.458 130.93841) (width 0.25) (layer F.Cu) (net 14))
 (segment (start 98.12 113.504759) (end 98.12 112.09) (width 0.25) (layer F.Cu) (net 13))
 (segment (start 98.45 111.76) (end 110.49 111.76) (width 0.25) (layer F.Cu) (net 13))
 (segment (start 98.12 112.09) (end 98.45 111.76) (width 0.25) (layer F.Cu) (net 13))
 (segment (start 111.577001 112.847001) (end 111.577001 127.182999) (width 0.25) (layer F.Cu) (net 13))
 (segment (start 111.577001 127.182999) (end 107.95 130.81) (width 0.25) (layer F.Cu) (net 13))
 (segment (start 110.49 111.76) (end 111.577001 112.847001) (width 0.25) (layer F.Cu) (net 13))
 (segment (start 107.95 130.81) (end 107.95 134.62) (width 0.25) (layer F.Cu) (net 13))
 (segment (start 109.728001 136.398001) (end 110.49 137.16) (width 0.25) (layer F.Cu) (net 13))
 (segment (start 107.95 134.62) (end 109.728001 136.398001) (width 0.25) (layer F.Cu) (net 13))
 (segment (start 98.12 118.104759) (end 98.12 116.51) (width 0.25) (layer F.Cu) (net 12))
 (segment (start 98.12 116.51) (end 99.06 115.57) (width 0.25) (layer F.Cu) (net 12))
 (segment (start 99.06 115.57) (end 104.14 115.57) (width 0.25) (layer F.Cu) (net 12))
 (segment (start 110.49 114.3) (end 105.41 114.3) (width 0.25) (layer F.Cu) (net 12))
 (segment (start 105.41 114.3) (end 104.14 115.57) (width 0.25) (layer F.Cu) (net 12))
 (segment (start 110.49 114.3) (end 113.03 114.3) (width 0.25) (layer B.Cu) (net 12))
 (segment (start 113.03 114.3) (end 115.57 116.84) (width 0.25) (layer B.Cu) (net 12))
 (segment (start 115.57 134.62) (end 110.49 139.7) (width 0.25) (layer B.Cu) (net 12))
 (segment (start 115.57 116.84) (end 115.57 134.62) (width 0.25) (layer B.Cu) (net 12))
 (segment (start 123.19 137.16) (end 129.54 137.16) (width 0.8) (layer F.Cu) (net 16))
 (segment (start 129.54 139.7) (end 123.19 139.7) (width 0.8) (layer F.Cu) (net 17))
 (segment (start 123.19 142.24) (end 129.54 142.24) (width 0.8) (layer F.Cu) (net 18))
 (segment (start 129.54 144.78) (end 123.19 144.78) (width 0.8) (layer F.Cu) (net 19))
 (segment (start 123.19 111.76) (end 129.54 111.76) (width 0.8) (layer F.Cu) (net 3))
 (segment (start 129.54 114.3) (end 123.19 114.3) (width 0.8) (layer F.Cu) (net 4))
 (segment (start 123.19 116.84) (end 129.54 116.84) (width 0.8) (layer F.Cu) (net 5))
 (segment (start 129.54 119.38) (end 123.19 119.38) (width 0.8) (layer F.Cu) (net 6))
 (segment (start 111.251999 107.441999) (end 110.49 106.68) (width 0.25) (layer F.Cu) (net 15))
 (segment (start 114.808 110.998) (end 111.251999 107.441999) (width 0.25) (layer F.Cu) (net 15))
 (segment (start 114.808 127.762) (end 114.808 110.998) (width 0.25) (layer F.Cu) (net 15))
 (segment (start 110.49 132.08) (end 114.808 127.762) (width 0.25) (layer F.Cu) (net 15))
 (segment (start 113.538 145.880762) (end 113.538 135.128) (width 0.25) (layer F.Cu) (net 15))
 (segment (start 111.011761 148.407001) (end 113.538 145.880762) (width 0.25) (layer F.Cu) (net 15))
 (segment (start 110.334237 148.407001) (end 111.011761 148.407001) (width 0.25) (layer F.Cu) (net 15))
 (segment (start 53.522999 140.787001) (end 53.522999 149.534999) (width 0.25) (layer F.Cu) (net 15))
 (segment (start 54.61 139.7) (end 53.522999 140.787001) (width 0.25) (layer F.Cu) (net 15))
 (segment (start 108.627238 150.114) (end 110.334237 148.407001) (width 0.25) (layer F.Cu) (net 15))
 (segment (start 113.538 135.128) (end 110.49 132.08) (width 0.25) (layer F.Cu) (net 15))
 (segment (start 53.522999 149.534999) (end 54.102 150.114) (width 0.25) (layer F.Cu) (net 15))
 (segment (start 54.102 150.114) (end 108.627238 150.114) (width 0.25) (layer F.Cu) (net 15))
 (segment (start 55.371999 126.238001) (end 54.61 127) (width 0.25) (layer F.Cu) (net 11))
 (segment (start 60.865001 120.744999) (end 55.371999 126.238001) (width 0.25) (layer F.Cu) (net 11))
 (segment (start 106.585001 120.744999) (end 60.865001 120.744999) (width 0.25) (layer F.Cu) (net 11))
 (segment (start 110.49 116.84) (end 106.585001 120.744999) (width 0.25) (layer F.Cu) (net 11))
 (segment (start 111.251999 117.601999) (end 110.49 116.84) (width 0.25) (layer B.Cu) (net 11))
 (segment (start 114.046 132.672762) (end 114.046 120.396) (width 0.25) (layer B.Cu) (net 11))
 (segment (start 107.95 139.7) (end 107.95 138.091238) (width 0.25) (layer B.Cu) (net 11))
 (segment (start 107.95 138.091238) (end 110.334237 135.707001) (width 0.25) (layer B.Cu) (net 11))
 (segment (start 110.49 142.24) (end 107.95 139.7) (width 0.25) (layer B.Cu) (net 11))
 (segment (start 111.011761 135.707001) (end 114.046 132.672762) (width 0.25) (layer B.Cu) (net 11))
 (segment (start 114.046 120.396) (end 111.251999 117.601999) (width 0.25) (layer B.Cu) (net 11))
 (segment (start 110.334237 135.707001) (end 111.011761 135.707001) (width 0.25) (layer B.Cu) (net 11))
 (segment (start 53.522999 125.547001) (end 53.848001 125.221999) (width 0.25) (layer F.Cu) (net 10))
 (segment (start 53.522999 127.521761) (end 53.522999 125.547001) (width 0.25) (layer F.Cu) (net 10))
 (segment (start 54.088239 128.087001) (end 53.522999 127.521761) (width 0.25) (layer F.Cu) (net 10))
 (segment (start 55.131761 128.087001) (end 54.088239 128.087001) (width 0.25) (layer F.Cu) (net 10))
 (segment (start 59.933763 123.284999) (end 55.131761 128.087001) (width 0.25) (layer F.Cu) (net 10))
 (segment (start 53.848001 125.221999) (end 54.61 124.46) (width 0.25) (layer F.Cu) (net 10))
 (segment (start 86.924001 123.284999) (end 59.933763 123.284999) (width 0.25) (layer F.Cu) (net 10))
 (segment (start 88.739009 121.469991) (end 86.924001 123.284999) (width 0.25) (layer F.Cu) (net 10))
 (segment (start 108.400009 121.469991) (end 88.739009 121.469991) (width 0.25) (layer F.Cu) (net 10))
 (segment (start 110.49 119.38) (end 108.400009 121.469991) (width 0.25) (layer F.Cu) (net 10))
 (segment (start 107.499991 122.370009) (end 109.728001 120.141999) (width 0.25) (layer B.Cu) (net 10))
 (segment (start 107.499991 140.858753) (end 107.499991 122.370009) (width 0.25) (layer B.Cu) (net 10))
 (segment (start 109.728001 120.141999) (end 110.49 119.38) (width 0.25) (layer B.Cu) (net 10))
 (segment (start 110.49 143.848762) (end 107.499991 140.858753) (width 0.25) (layer B.Cu) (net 10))
 (segment (start 110.49 144.78) (end 110.49 143.848762) (width 0.25) (layer B.Cu) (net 10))
 (segment (start 123.19 121.92) (end 121.92 121.92) (width 0.25) (layer F.Cu) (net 7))
 (segment (start 121.902999 121.902999) (end 120.632999 121.902999) (width 0.25) (layer F.Cu) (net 7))
 (segment (start 121.92 121.92) (end 121.902999 121.902999) (width 0.25) (layer F.Cu) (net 7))
 (segment (start 120.632999 121.902999) (end 118.11 119.38) (width 0.25) (layer F.Cu) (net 7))
 (segment (start 118.11 119.38) (end 118.11 105.41) (width 0.25) (layer F.Cu) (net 7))
 (segment (start 118.11 105.41) (end 116.84 104.14) (width 0.25) (layer F.Cu) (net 7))
 (segment (start 67.31 104.14) (end 54.61 116.84) (width 0.25) (layer F.Cu) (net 7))
 (segment (start 116.84 104.14) (end 67.31 104.14) (width 0.25) (layer F.Cu) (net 7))
 (segment (start 123.19 147.32) (end 119.38 147.32) (width 0.25) (layer F.Cu) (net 20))
 (segment (start 119.38 147.32) (end 117.927001 148.772999) (width 0.25) (layer F.Cu) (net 20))
 (segment (start 107.611238 151.13) (end 57.010108 151.13) (width 0.25) (layer F.Cu) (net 20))
 (segment (start 57.010108 151.13) (end 53.34 151.13) (width 0.25) (layer F.Cu) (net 20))
 (segment (start 53.34 151.13) (end 52.07 149.86) (width 0.25) (layer F.Cu) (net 20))
 (segment (start 52.07 149.86) (end 52.07 116.64113) (width 0.25) (layer F.Cu) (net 20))
 (segment (start 52.07 116.64113) (end 52.07 115.57) (width 0.25) (layer F.Cu) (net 20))
 (segment (start 53.53237 114.10113) (end 52.07 115.5635) (width 0.25) (layer F.Cu) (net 20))
 (segment (start 54.61 114.10113) (end 53.53237 114.10113) (width 0.25) (layer F.Cu) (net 20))
 (segment (start 107.611238 151.13) (end 115.57 151.13) (width 0.25) (layer F.Cu) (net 20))
 (segment (start 115.57 151.13) (end 118.11 148.59) (width 0.25) (layer F.Cu) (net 20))
 (segment (start 80.771999 123.698001) (end 80.01 124.46) (width 0.25) (layer B.Cu) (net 22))
 (segment (start 81.185001 123.284999) (end 80.771999 123.698001) (width 0.25) (layer B.Cu) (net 22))
 (segment (start 88.740001 123.284999) (end 81.185001 123.284999) (width 0.25) (layer B.Cu) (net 22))
 (segment (start 109.402999 143.947997) (end 88.740001 123.284999) (width 0.25) (layer B.Cu) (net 22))
 (segment (start 109.402999 146.232999) (end 109.402999 143.947997) (width 0.25) (layer B.Cu) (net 22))
 (segment (start 110.49 147.32) (end 109.402999 146.232999) (width 0.25) (layer B.Cu) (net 22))
 (segment (start 80.771999 126.238001) (end 80.01 127) (width 0.25) (layer B.Cu) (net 21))
 (segment (start 100.235001 136.595999) (end 89.464001 125.824999) (width 0.25) (layer B.Cu) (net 21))
 (segment (start 89.464001 125.824999) (end 81.185001 125.824999) (width 0.25) (layer B.Cu) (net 21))
 (segment (start 100.235001 139.350003) (end 100.235001 136.595999) (width 0.25) (layer B.Cu) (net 21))
 (segment (start 101.759999 140.875001) (end 100.235001 139.350003) (width 0.25) (layer B.Cu) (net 21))
 (segment (start 103.244003 140.875001) (end 101.759999 140.875001) (width 0.25) (layer B.Cu) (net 21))
 (segment (start 104.045001 143.415001) (end 104.045001 141.675999) (width 0.25) (layer B.Cu) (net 21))
 (segment (start 81.185001 125.824999) (end 80.771999 126.238001) (width 0.25) (layer B.Cu) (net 21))
 (segment (start 104.045001 141.675999) (end 103.244003 140.875001) (width 0.25) (layer B.Cu) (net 21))
 (segment (start 110.49 149.86) (end 104.045001 143.415001) (width 0.25) (layer B.Cu) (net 21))
 (segment (start 102.87 121.92) (end 88.9 135.89) (width 0.25) (layer F.Cu) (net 9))
 (segment (start 110.49 121.92) (end 102.87 121.92) (width 0.25) (layer F.Cu) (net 9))
 (segment (start 83.82 135.89) (end 80.01 132.08) (width 0.25) (layer F.Cu) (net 9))
 (segment (start 88.9 135.89) (end 83.82 135.89) (width 0.25) (layer F.Cu) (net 9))
 (segment (start 110.49 124.46) (end 101.6 124.46) (width 0.25) (layer F.Cu) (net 8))
 (segment (start 101.6 124.46) (end 88.9 137.16) (width 0.25) (layer F.Cu) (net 8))
 (segment (start 88.9 137.16) (end 82.55 137.16) (width 0.25) (layer F.Cu) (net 8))
 (segment (start 82.55 137.16) (end 80.01 134.62) (width 0.25) (layer F.Cu) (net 8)))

